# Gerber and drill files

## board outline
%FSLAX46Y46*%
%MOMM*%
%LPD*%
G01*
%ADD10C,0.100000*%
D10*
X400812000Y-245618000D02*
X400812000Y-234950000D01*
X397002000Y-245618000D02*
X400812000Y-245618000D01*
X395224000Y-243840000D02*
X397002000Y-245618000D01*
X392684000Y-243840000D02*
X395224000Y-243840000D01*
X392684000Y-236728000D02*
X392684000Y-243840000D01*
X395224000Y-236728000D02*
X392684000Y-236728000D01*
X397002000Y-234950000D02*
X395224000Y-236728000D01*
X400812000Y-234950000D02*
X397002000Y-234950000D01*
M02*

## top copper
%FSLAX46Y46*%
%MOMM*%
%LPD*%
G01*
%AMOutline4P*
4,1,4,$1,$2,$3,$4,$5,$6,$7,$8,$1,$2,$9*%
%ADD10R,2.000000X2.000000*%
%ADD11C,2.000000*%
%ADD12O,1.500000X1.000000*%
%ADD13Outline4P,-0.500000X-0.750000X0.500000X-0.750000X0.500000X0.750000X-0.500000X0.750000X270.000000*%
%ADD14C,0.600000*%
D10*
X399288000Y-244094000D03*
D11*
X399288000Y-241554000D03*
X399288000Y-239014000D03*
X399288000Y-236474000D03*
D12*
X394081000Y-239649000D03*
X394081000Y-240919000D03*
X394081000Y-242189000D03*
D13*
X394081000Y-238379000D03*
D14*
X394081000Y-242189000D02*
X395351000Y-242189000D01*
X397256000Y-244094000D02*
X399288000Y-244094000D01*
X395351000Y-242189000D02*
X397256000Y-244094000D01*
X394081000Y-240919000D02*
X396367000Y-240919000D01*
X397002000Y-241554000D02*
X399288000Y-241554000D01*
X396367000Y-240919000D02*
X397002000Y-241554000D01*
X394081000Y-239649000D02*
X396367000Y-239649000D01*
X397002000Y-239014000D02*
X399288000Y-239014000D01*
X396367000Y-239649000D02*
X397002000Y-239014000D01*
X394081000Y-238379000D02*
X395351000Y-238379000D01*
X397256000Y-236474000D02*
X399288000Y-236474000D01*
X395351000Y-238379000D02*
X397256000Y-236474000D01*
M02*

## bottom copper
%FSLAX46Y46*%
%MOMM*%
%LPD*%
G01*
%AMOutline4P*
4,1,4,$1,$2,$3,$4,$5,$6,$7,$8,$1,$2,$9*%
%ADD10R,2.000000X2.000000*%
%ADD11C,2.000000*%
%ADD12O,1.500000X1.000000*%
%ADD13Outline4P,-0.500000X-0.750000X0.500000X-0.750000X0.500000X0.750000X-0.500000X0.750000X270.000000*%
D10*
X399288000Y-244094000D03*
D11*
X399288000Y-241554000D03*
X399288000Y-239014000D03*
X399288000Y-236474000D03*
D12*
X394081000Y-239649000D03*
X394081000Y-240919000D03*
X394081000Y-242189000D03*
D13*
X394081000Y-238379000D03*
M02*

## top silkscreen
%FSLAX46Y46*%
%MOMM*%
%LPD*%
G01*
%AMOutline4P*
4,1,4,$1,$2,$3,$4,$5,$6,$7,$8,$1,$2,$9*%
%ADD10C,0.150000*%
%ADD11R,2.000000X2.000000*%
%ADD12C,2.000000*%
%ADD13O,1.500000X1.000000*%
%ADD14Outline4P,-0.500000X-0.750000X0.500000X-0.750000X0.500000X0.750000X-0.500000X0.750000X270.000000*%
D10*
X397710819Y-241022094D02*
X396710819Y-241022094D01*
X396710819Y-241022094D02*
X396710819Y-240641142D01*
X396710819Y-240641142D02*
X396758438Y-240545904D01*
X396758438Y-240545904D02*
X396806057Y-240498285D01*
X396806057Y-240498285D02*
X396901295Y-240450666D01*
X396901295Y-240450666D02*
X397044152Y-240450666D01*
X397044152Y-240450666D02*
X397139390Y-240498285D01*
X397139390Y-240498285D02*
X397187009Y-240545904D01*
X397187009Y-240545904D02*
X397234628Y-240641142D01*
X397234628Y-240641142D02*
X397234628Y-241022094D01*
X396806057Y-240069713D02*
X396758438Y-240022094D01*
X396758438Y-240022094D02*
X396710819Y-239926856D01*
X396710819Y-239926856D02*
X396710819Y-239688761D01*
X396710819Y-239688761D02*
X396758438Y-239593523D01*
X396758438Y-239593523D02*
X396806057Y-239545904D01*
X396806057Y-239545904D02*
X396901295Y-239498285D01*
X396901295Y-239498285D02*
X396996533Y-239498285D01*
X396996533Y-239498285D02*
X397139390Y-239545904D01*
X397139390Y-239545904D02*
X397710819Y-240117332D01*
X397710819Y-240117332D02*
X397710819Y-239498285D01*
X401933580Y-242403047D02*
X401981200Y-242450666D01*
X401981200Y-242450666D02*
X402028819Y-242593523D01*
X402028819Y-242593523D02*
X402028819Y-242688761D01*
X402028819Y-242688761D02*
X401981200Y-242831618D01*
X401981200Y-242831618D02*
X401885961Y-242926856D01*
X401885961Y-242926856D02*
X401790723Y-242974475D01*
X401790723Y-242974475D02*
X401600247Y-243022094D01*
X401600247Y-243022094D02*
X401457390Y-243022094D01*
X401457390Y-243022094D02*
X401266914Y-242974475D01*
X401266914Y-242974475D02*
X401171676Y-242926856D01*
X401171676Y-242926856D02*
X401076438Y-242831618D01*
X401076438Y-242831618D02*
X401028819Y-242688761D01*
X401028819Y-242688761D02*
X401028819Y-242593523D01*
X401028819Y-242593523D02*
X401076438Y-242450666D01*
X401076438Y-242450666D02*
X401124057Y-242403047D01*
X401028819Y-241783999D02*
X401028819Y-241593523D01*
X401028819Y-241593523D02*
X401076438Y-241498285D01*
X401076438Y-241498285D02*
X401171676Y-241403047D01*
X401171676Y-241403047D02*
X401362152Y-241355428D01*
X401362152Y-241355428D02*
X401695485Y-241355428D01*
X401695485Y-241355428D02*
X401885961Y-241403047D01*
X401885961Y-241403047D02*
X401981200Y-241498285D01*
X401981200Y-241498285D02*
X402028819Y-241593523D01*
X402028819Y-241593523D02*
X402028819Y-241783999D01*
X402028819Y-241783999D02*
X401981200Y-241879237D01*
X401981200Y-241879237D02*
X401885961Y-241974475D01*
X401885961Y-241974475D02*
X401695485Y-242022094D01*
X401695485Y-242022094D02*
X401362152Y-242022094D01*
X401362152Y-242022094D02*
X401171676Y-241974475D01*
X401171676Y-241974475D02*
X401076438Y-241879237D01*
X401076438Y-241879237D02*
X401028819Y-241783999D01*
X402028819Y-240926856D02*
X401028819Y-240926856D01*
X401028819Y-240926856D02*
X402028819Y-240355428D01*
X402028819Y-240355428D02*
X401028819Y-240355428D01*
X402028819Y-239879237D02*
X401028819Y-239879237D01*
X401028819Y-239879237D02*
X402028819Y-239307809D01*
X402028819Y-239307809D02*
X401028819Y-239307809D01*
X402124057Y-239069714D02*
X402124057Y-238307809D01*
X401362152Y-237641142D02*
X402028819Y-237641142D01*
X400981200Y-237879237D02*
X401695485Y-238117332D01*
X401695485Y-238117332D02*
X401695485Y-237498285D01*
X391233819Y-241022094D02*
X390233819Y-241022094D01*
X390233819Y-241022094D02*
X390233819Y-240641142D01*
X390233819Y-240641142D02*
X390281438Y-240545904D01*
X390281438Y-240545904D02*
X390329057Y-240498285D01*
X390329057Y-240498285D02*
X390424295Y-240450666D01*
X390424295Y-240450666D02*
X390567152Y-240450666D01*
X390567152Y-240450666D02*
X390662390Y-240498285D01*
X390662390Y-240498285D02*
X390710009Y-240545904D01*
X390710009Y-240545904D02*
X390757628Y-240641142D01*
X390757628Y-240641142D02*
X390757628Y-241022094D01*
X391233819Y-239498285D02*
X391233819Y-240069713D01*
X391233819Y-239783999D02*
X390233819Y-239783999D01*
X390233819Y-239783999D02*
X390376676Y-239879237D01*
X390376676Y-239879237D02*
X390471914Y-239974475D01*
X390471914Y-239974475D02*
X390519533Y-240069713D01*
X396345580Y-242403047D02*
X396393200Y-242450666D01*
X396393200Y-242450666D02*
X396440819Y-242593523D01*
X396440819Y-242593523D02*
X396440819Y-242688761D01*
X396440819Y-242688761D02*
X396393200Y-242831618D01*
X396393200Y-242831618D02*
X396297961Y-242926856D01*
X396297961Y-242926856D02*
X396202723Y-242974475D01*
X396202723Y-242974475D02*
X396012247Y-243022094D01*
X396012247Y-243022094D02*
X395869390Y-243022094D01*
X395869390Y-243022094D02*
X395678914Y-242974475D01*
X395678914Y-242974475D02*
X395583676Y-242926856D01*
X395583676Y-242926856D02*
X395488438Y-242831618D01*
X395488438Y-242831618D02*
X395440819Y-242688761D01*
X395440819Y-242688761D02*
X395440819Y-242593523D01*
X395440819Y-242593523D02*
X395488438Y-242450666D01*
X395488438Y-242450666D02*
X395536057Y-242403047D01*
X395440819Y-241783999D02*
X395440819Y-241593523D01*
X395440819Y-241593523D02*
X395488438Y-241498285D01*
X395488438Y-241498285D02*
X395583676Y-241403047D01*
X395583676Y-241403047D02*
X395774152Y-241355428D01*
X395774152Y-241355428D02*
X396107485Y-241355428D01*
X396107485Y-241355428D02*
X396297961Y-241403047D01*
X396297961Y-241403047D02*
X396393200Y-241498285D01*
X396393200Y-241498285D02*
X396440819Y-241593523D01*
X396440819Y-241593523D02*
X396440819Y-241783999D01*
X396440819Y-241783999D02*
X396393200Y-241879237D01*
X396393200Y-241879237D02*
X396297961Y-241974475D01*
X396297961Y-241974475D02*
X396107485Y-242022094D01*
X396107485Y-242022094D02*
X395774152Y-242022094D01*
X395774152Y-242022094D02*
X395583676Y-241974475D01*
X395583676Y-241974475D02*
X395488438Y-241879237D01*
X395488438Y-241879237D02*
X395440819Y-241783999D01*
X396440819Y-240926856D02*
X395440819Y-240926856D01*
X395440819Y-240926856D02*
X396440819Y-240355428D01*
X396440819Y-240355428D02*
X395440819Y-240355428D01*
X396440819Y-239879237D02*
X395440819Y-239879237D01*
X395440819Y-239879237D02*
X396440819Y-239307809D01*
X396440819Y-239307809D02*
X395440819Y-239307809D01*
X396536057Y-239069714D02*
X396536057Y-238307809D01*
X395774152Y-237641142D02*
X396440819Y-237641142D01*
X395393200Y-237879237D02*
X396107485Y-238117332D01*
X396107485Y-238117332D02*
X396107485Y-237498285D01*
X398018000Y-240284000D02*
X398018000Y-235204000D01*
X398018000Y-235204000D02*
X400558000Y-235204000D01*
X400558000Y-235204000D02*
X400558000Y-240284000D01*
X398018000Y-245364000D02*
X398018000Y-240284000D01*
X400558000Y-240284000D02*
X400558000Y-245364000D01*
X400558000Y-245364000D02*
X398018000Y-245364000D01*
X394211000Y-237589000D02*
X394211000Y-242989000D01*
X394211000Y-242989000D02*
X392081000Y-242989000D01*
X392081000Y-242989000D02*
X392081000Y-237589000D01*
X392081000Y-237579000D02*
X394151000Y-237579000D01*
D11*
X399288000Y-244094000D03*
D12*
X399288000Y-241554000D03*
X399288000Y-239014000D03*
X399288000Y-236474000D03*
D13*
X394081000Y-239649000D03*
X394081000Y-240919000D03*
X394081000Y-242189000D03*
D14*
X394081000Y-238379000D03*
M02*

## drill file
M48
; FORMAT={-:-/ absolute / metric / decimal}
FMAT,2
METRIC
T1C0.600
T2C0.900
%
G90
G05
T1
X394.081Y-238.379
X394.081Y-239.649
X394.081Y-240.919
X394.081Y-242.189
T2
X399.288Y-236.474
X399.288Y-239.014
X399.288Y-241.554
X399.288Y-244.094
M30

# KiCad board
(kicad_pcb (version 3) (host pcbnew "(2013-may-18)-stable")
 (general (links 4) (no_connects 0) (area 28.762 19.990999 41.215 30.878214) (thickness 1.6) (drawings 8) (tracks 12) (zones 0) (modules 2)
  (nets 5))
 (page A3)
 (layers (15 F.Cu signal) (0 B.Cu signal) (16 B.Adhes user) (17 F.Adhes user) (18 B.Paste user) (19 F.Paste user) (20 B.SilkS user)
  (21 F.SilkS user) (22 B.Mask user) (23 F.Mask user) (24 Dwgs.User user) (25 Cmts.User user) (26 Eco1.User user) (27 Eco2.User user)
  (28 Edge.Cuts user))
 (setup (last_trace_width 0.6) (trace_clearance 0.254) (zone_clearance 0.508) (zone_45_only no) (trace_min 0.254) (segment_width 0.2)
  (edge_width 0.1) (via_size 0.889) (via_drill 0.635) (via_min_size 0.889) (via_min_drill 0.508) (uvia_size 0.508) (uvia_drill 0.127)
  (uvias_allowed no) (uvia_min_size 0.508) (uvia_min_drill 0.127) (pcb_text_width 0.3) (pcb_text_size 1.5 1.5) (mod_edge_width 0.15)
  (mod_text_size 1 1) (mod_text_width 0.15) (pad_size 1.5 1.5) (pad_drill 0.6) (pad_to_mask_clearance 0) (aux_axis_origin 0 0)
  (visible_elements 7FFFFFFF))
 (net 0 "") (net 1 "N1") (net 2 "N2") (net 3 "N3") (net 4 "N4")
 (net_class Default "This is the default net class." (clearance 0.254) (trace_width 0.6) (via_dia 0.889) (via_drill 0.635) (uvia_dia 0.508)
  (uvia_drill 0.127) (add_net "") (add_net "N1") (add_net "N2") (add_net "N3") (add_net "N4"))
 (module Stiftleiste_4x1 (layer F.Cu) (at 399.288 240.284 90)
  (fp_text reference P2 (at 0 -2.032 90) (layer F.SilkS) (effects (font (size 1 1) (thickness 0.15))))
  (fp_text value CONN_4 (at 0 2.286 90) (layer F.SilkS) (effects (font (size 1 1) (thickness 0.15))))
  (fp_line (start 0 -1.27) (end 5.08 -1.27) (layer F.SilkS) (width 0.15))
  (fp_line (start 5.08 -1.27) (end 5.08 1.27) (layer F.SilkS) (width 0.15))
  (fp_line (start 5.08 1.27) (end 0 1.27) (layer F.SilkS) (width 0.15))
  (fp_line (start -5.08 -1.27) (end 0 -1.27) (layer F.SilkS) (width 0.15))
  (fp_line (start 0 1.27) (end -5.08 1.27) (layer F.SilkS) (width 0.15))
  (fp_line (start -5.08 1.27) (end -5.08 -1.27) (layer F.SilkS) (width 0.15))
  (pad 1 thru_hole rect (at -3.81 0 90) (size 2 2) (drill 0.9) (layers *.Cu *.Mask F.SilkS) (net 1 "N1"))
  (pad 2 thru_hole circle (at -1.27 0 90) (size 2 2) (drill 0.9) (layers *.Cu *.Mask F.SilkS) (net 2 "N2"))
  (pad 3 thru_hole circle (at 1.27 0 90) (size 2 2) (drill 0.9) (layers *.Cu *.Mask F.SilkS) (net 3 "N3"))
  (pad 4 thru_hole circle (at 3.81 0 90) (size 2 2) (drill 0.9) (layers *.Cu *.Mask F.SilkS) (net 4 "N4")))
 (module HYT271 (layer F.Cu) (at 394.208 240.284 270)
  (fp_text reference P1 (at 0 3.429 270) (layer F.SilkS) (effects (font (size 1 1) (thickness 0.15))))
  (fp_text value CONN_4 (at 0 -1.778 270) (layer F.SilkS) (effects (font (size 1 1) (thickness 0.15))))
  (fp_line (start -2.695 -0.003) (end 2.705 -0.003) (layer F.SilkS) (width 0.15))
  (fp_line (start 2.705 -0.003) (end 2.705 2.127) (layer F.SilkS) (width 0.15))
  (fp_line (start 2.705 2.127) (end -2.695 2.127) (layer F.SilkS) (width 0.15))
  (fp_line (start -2.705 2.127) (end -2.705 0.057) (layer F.SilkS) (width 0.15))
  (pad 2 thru_hole oval (at -0.635 0.127 270) (size 1 1.5) (drill 0.6) (layers *.Cu *.Mask F.SilkS) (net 3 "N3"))
  (pad 3 thru_hole oval (at 0.635 0.127 270) (size 1 1.5) (drill 0.6) (layers *.Cu *.Mask F.SilkS) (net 2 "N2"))
  (pad 4 thru_hole oval (at 1.905 0.127 270) (size 1 1.5) (drill 0.6) (layers *.Cu *.Mask F.SilkS) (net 1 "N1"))
  (pad 1 thru_hole trapezoid (at -1.905 0.127 270) (size 1 1.5) (drill 0.6) (layers *.Cu *.Mask F.SilkS) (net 4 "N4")))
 (gr_line (start 400.812 245.618) (end 400.812 234.95) (angle 90) (layer Edge.Cuts) (width 0.1))
 (gr_line (start 397.002 245.618) (end 400.812 245.618) (angle 90) (layer Edge.Cuts) (width 0.1))
 (gr_line (start 395.224 243.84) (end 397.002 245.618) (angle 90) (layer Edge.Cuts) (width 0.1))
 (gr_line (start 392.684 243.84) (end 395.224 243.84) (angle 90) (layer Edge.Cuts) (width 0.1))
 (gr_line (start 392.684 236.728) (end 392.684 243.84) (angle 90) (layer Edge.Cuts) (width 0.1))
 (gr_line (start 395.224 236.728) (end 392.684 236.728) (angle 90) (layer Edge.Cuts) (width 0.1))
 (gr_line (start 397.002 234.95) (end 395.224 236.728) (angle 90) (layer Edge.Cuts) (width 0.1))
 (gr_line (start 400.812 234.95) (end 397.002 234.95) (angle 90) (layer Edge.Cuts) (width 0.1))
 (segment (start 394.081 242.189) (end 395.351 242.189) (width 0.6) (layer F.Cu) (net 1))
 (segment (start 397.256 244.094) (end 399.288 244.094) (width 0.6) (layer F.Cu) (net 1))
 (segment (start 395.351 242.189) (end 397.256 244.094) (width 0.6) (layer F.Cu) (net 1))
 (segment (start 394.081 240.919) (end 396.367 240.919) (width 0.6) (layer F.Cu) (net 2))
 (segment (start 397.002 241.554) (end 399.288 241.554) (width 0.6) (layer F.Cu) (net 2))
 (segment (start 396.367 240.919) (end 397.002 241.554) (width 0.6) (layer F.Cu) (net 2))
 (segment (start 394.081 239.649) (end 396.367 239.649) (width 0.6) (layer F.Cu) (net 3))
 (segment (start 397.002 239.014) (end 399.288 239.014) (width 0.6) (layer F.Cu) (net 3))
 (segment (start 396.367 239.649) (end 397.002 239.014) (width 0.6) (layer F.Cu) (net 3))
 (segment (start 394.081 238.379) (end 395.351 238.379) (width 0.6) (layer F.Cu) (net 4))
 (segment (start 397.256 236.474) (end 399.288 236.474) (width 0.6) (layer F.Cu) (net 4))
 (segment (start 395.351 238.379) (end 397.256 236.474) (width 0.6) (layer F.Cu) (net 4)))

